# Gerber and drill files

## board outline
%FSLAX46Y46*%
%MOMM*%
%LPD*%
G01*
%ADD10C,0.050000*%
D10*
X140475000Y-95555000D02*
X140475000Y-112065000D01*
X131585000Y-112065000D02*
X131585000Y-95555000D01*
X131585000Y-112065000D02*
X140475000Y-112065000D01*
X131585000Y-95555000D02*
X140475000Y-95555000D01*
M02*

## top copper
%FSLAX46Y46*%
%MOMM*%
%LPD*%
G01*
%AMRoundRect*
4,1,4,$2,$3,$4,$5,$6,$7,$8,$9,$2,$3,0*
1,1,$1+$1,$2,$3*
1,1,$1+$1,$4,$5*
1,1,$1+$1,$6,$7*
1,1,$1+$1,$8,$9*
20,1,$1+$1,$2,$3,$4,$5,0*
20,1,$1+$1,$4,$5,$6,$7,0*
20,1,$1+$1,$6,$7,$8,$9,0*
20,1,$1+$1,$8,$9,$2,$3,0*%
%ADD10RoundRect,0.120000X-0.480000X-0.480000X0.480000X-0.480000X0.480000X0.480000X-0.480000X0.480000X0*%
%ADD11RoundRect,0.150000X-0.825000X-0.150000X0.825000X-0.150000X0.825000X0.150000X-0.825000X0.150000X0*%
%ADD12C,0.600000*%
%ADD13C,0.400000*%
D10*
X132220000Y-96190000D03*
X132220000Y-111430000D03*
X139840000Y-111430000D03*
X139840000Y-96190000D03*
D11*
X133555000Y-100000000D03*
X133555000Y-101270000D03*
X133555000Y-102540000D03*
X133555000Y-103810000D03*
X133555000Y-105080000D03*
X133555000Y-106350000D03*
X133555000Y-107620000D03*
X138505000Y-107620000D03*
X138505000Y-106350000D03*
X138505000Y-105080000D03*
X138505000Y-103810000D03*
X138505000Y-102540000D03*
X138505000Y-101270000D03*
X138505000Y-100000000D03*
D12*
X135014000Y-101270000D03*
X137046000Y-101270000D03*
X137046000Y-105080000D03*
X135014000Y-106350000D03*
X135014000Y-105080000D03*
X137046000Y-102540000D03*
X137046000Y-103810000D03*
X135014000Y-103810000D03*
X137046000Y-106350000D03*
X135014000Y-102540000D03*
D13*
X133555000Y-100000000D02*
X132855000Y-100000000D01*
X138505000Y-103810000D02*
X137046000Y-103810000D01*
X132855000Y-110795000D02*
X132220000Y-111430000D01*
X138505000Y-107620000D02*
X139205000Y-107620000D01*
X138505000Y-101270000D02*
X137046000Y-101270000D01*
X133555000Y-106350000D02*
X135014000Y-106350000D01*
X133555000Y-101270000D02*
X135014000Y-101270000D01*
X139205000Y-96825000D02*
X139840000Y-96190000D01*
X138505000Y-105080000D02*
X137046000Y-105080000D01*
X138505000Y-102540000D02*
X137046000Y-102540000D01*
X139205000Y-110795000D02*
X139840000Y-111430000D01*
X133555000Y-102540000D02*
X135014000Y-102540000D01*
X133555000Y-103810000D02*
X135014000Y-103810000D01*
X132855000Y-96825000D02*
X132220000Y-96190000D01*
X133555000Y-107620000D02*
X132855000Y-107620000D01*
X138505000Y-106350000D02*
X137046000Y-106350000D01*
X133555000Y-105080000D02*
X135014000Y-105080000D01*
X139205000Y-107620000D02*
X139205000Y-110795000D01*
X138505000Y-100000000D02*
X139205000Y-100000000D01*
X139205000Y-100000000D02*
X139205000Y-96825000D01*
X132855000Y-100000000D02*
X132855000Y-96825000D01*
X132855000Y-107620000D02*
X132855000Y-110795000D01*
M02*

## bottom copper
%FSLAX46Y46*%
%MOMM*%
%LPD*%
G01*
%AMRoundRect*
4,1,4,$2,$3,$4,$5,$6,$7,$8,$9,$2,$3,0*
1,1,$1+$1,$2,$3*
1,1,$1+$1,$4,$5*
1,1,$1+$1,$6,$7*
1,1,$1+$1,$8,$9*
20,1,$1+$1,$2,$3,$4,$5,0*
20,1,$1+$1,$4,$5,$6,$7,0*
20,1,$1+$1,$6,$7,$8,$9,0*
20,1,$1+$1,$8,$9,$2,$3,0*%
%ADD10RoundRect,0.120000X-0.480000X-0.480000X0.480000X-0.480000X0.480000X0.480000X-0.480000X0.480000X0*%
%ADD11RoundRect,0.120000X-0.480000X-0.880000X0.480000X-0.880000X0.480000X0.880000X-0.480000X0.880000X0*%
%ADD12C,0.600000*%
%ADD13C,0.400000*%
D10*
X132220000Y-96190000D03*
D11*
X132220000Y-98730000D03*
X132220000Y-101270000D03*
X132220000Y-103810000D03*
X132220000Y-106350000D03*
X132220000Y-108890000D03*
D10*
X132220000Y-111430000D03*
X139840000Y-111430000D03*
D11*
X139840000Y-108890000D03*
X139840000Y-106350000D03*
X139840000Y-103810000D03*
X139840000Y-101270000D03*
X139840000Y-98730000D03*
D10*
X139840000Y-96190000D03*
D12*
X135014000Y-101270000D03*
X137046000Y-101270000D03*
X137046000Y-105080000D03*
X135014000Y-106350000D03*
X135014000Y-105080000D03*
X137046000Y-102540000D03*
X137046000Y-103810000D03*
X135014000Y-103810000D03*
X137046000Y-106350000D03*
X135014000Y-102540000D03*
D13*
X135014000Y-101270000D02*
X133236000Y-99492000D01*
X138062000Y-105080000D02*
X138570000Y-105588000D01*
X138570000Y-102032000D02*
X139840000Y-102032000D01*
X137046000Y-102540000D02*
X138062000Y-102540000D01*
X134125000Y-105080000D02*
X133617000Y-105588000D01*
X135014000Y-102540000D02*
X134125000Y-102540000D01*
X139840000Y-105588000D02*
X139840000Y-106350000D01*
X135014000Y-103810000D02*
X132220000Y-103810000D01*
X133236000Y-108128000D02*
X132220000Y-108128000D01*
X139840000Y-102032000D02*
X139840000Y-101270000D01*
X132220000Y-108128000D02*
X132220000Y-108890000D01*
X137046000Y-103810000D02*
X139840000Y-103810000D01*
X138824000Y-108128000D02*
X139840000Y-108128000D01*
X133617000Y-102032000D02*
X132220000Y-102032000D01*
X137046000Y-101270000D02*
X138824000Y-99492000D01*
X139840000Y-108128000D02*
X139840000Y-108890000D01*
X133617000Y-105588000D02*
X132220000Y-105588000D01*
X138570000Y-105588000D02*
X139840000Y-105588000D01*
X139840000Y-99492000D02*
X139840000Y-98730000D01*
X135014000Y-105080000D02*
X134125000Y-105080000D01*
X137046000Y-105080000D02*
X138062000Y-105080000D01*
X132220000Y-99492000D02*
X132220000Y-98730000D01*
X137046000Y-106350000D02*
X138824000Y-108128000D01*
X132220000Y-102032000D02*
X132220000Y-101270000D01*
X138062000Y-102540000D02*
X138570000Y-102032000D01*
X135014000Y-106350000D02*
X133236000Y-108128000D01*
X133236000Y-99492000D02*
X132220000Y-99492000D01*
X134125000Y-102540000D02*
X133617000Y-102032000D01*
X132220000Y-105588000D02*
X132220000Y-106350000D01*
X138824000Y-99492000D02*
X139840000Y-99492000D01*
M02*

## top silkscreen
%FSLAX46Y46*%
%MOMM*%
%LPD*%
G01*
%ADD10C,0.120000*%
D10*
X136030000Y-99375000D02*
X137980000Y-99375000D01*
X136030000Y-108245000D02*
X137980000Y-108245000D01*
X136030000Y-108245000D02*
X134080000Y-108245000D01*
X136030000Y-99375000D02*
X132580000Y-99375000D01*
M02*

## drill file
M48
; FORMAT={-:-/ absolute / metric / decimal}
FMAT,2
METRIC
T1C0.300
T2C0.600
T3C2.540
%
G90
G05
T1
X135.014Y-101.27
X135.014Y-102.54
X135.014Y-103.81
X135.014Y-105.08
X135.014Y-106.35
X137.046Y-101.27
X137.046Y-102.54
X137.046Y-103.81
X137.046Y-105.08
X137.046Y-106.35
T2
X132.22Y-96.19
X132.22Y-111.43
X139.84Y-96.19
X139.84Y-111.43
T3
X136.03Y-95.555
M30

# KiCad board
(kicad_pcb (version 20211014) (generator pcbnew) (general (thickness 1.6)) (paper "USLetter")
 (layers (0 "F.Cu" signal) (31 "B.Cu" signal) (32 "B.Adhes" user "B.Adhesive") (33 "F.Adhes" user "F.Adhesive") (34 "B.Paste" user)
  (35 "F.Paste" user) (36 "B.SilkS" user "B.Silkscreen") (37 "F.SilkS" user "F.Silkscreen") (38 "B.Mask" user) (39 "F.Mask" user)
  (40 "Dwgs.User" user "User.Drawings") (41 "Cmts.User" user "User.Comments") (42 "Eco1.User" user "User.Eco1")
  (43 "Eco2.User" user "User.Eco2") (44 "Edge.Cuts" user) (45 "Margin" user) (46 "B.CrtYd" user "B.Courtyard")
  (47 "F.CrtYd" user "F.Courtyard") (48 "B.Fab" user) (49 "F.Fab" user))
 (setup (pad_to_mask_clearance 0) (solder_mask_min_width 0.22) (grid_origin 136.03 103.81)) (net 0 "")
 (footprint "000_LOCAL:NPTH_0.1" (layer "F.Cu") (at 136.03 95.555)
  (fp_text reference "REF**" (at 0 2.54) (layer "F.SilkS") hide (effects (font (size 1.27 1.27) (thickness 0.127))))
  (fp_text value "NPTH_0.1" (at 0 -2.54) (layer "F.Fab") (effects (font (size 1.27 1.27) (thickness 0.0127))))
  (pad "" np_thru_hole circle locked (at 0 0) (size 2.54 2.54) (drill 2.54) (layers *.Cu *.Mask)))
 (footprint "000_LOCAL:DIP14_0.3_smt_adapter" (layer "F.Cu") (at 136.03 103.81)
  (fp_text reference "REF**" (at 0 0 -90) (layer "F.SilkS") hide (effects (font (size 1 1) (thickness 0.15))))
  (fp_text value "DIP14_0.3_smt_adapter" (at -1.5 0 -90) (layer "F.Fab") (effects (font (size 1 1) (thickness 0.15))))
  (pad "1" thru_hole roundrect locked (at -3.81 -7.62) (size 1.2 1.2) (drill 0.6) (layers *.Cu *.Mask) (roundrect_rratio 0.1))
  (pad "2" smd roundrect locked (at -3.81 -5.08) (size 1.2 2) (layers "B.Cu" "B.Mask") (roundrect_rratio 0.1))
  (pad "3" smd roundrect locked (at -3.81 -2.54) (size 1.2 2) (layers "B.Cu" "B.Mask") (roundrect_rratio 0.1))
  (pad "4" smd roundrect locked (at -3.81 0) (size 1.2 2) (layers "B.Cu" "B.Mask") (roundrect_rratio 0.1))
  (pad "5" smd roundrect locked (at -3.81 2.54) (size 1.2 2) (layers "B.Cu" "B.Mask") (roundrect_rratio 0.1))
  (pad "6" smd roundrect locked (at -3.81 5.08) (size 1.2 2) (layers "B.Cu" "B.Mask") (roundrect_rratio 0.1))
  (pad "7" thru_hole roundrect locked (at -3.81 7.62) (size 1.2 1.2) (drill 0.6) (layers *.Cu *.Mask) (roundrect_rratio 0.1))
  (pad "8" thru_hole roundrect locked (at 3.81 7.62) (size 1.2 1.2) (drill 0.6) (layers *.Cu *.Mask) (roundrect_rratio 0.1))
  (pad "9" smd roundrect locked (at 3.81 5.08) (size 1.2 2) (layers "B.Cu" "B.Mask") (roundrect_rratio 0.1))
  (pad "10" smd roundrect locked (at 3.81 2.54) (size 1.2 2) (layers "B.Cu" "B.Mask") (roundrect_rratio 0.1))
  (pad "11" smd roundrect locked (at 3.81 0) (size 1.2 2) (layers "B.Cu" "B.Mask") (roundrect_rratio 0.1))
  (pad "12" smd roundrect locked (at 3.81 -2.54) (size 1.2 2) (layers "B.Cu" "B.Mask") (roundrect_rratio 0.1))
  (pad "13" smd roundrect locked (at 3.81 -5.08) (size 1.2 2) (layers "B.Cu" "B.Mask") (roundrect_rratio 0.1))
  (pad "14" thru_hole roundrect locked (at 3.81 -7.62) (size 1.2 1.2) (drill 0.6) (layers *.Cu *.Mask) (roundrect_rratio 0.1)))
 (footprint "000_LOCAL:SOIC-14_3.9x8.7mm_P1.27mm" (layer "F.Cu") (at 136.03 103.81)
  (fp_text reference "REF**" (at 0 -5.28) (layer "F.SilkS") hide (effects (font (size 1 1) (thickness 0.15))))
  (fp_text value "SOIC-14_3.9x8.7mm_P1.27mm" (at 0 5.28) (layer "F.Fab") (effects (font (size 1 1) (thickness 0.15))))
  (fp_line (start 0 -4.435) (end 1.95 -4.435) (layer "F.SilkS") (width 0.12))
  (fp_line (start 0 4.435) (end 1.95 4.435) (layer "F.SilkS") (width 0.12))
  (fp_line (start 0 4.435) (end -1.95 4.435) (layer "F.SilkS") (width 0.12))
  (fp_line (start 0 -4.435) (end -3.45 -4.435) (layer "F.SilkS") (width 0.12))
  (pad "1" smd roundrect locked (at -2.475 -3.81) (size 1.95 0.6) (layers "F.Cu" "F.Paste" "F.Mask") (roundrect_rratio 0.25))
  (pad "2" smd roundrect locked (at -2.475 -2.54) (size 1.95 0.6) (layers "F.Cu" "F.Paste" "F.Mask") (roundrect_rratio 0.25))
  (pad "3" smd roundrect locked (at -2.475 -1.27) (size 1.95 0.6) (layers "F.Cu" "F.Paste" "F.Mask") (roundrect_rratio 0.25))
  (pad "4" smd roundrect locked (at -2.475 0) (size 1.95 0.6) (layers "F.Cu" "F.Paste" "F.Mask") (roundrect_rratio 0.25))
  (pad "5" smd roundrect locked (at -2.475 1.27) (size 1.95 0.6) (layers "F.Cu" "F.Paste" "F.Mask") (roundrect_rratio 0.25))
  (pad "6" smd roundrect locked (at -2.475 2.54) (size 1.95 0.6) (layers "F.Cu" "F.Paste" "F.Mask") (roundrect_rratio 0.25))
  (pad "7" smd roundrect locked (at -2.475 3.81) (size 1.95 0.6) (layers "F.Cu" "F.Paste" "F.Mask") (roundrect_rratio 0.25))
  (pad "8" smd roundrect locked (at 2.475 3.81) (size 1.95 0.6) (layers "F.Cu" "F.Paste" "F.Mask") (roundrect_rratio 0.25))
  (pad "9" smd roundrect locked (at 2.475 2.54) (size 1.95 0.6) (layers "F.Cu" "F.Paste" "F.Mask") (roundrect_rratio 0.25))
  (pad "10" smd roundrect locked (at 2.475 1.27) (size 1.95 0.6) (layers "F.Cu" "F.Paste" "F.Mask") (roundrect_rratio 0.25))
  (pad "11" smd roundrect locked (at 2.475 0) (size 1.95 0.6) (layers "F.Cu" "F.Paste" "F.Mask") (roundrect_rratio 0.25))
  (pad "12" smd roundrect locked (at 2.475 -1.27) (size 1.95 0.6) (layers "F.Cu" "F.Paste" "F.Mask") (roundrect_rratio 0.25))
  (pad "13" smd roundrect locked (at 2.475 -2.54) (size 1.95 0.6) (layers "F.Cu" "F.Paste" "F.Mask") (roundrect_rratio 0.25))
  (pad "14" smd roundrect locked (at 2.475 -3.81) (size 1.95 0.6) (layers "F.Cu" "F.Paste" "F.Mask") (roundrect_rratio 0.25)))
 (gr_line (start 140.475 95.555) (end 140.475 112.065) (layer "Edge.Cuts") (width 0.05))
 (gr_line (start 131.585 112.065) (end 131.585 95.555) (layer "Edge.Cuts") (width 0.05))
 (gr_line (start 131.585 112.065) (end 140.475 112.065) (layer "Edge.Cuts") (width 0.05))
 (gr_line (start 131.585 95.555) (end 140.475 95.555) (layer "Edge.Cuts") (width 0.05))
 (segment (start 133.555 100) (end 132.855 100) (width 0.4) (layer "F.Cu") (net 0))
 (segment (start 138.505 103.81) (end 137.046 103.81) (width 0.4) (layer "F.Cu") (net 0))
 (segment (start 132.855 110.795) (end 132.22 111.43) (width 0.4) (layer "F.Cu") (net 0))
 (segment (start 138.505 107.62) (end 139.205 107.62) (width 0.4) (layer "F.Cu") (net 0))
 (segment (start 138.505 101.27) (end 137.046 101.27) (width 0.4) (layer "F.Cu") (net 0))
 (segment (start 133.555 106.35) (end 135.014 106.35) (width 0.4) (layer "F.Cu") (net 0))
 (segment (start 133.555 101.27) (end 135.014 101.27) (width 0.4) (layer "F.Cu") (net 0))
 (segment (start 139.205 96.825) (end 139.84 96.19) (width 0.4) (layer "F.Cu") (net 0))
 (segment (start 138.505 105.08) (end 137.046 105.08) (width 0.4) (layer "F.Cu") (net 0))
 (segment (start 138.505 102.54) (end 137.046 102.54) (width 0.4) (layer "F.Cu") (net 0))
 (segment (start 139.205 110.795) (end 139.84 111.43) (width 0.4) (layer "F.Cu") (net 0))
 (segment (start 133.555 102.54) (end 135.014 102.54) (width 0.4) (layer "F.Cu") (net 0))
 (segment (start 133.555 103.81) (end 135.014 103.81) (width 0.4) (layer "F.Cu") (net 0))
 (segment (start 132.855 96.825) (end 132.22 96.19) (width 0.4) (layer "F.Cu") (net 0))
 (segment (start 133.555 107.62) (end 132.855 107.62) (width 0.4) (layer "F.Cu") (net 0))
 (segment (start 138.505 106.35) (end 137.046 106.35) (width 0.4) (layer "F.Cu") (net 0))
 (segment (start 133.555 105.08) (end 135.014 105.08) (width 0.4) (layer "F.Cu") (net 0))
 (segment (start 139.205 107.62) (end 139.205 110.795) (width 0.4) (layer "F.Cu") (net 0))
 (segment (start 138.505 100) (end 139.205 100) (width 0.4) (layer "F.Cu") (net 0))
 (segment (start 139.205 100) (end 139.205 96.825) (width 0.4) (layer "F.Cu") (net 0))
 (segment (start 132.855 100) (end 132.855 96.825) (width 0.4) (layer "F.Cu") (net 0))
 (segment (start 132.855 107.62) (end 132.855 110.795) (width 0.4) (layer "F.Cu") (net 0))
 (via (at 135.014 101.27) (size 0.6) (drill 0.3) (layers "F.Cu" "B.Cu") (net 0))
 (via (at 137.046 101.27) (size 0.6) (drill 0.3) (layers "F.Cu" "B.Cu") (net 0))
 (via (at 137.046 105.08) (size 0.6) (drill 0.3) (layers "F.Cu" "B.Cu") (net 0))
 (via (at 135.014 106.35) (size 0.6) (drill 0.3) (layers "F.Cu" "B.Cu") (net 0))
 (via (at 135.014 105.08) (size 0.6) (drill 0.3) (layers "F.Cu" "B.Cu") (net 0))
 (via (at 137.046 102.54) (size 0.6) (drill 0.3) (layers "F.Cu" "B.Cu") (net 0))
 (via (at 137.046 103.81) (size 0.6) (drill 0.3) (layers "F.Cu" "B.Cu") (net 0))
 (via (at 135.014 103.81) (size 0.6) (drill 0.3) (layers "F.Cu" "B.Cu") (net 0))
 (via (at 137.046 106.35) (size 0.6) (drill 0.3) (layers "F.Cu" "B.Cu") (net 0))
 (via (at 135.014 102.54) (size 0.6) (drill 0.3) (layers "F.Cu" "B.Cu") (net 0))
 (segment (start 135.014 101.27) (end 133.236 99.492) (width 0.4) (layer "B.Cu") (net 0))
 (segment (start 138.062 105.08) (end 138.57 105.588) (width 0.4) (layer "B.Cu") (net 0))
 (segment (start 138.57 102.032) (end 139.84 102.032) (width 0.4) (layer "B.Cu") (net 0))
 (segment (start 137.046 102.54) (end 138.062 102.54) (width 0.4) (layer "B.Cu") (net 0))
 (segment (start 134.125 105.08) (end 133.617 105.588) (width 0.4) (layer "B.Cu") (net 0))
 (segment (start 135.014 102.54) (end 134.125 102.54) (width 0.4) (layer "B.Cu") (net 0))
 (segment (start 139.84 105.588) (end 139.84 106.35) (width 0.4) (layer "B.Cu") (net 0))
 (segment (start 135.014 103.81) (end 132.22 103.81) (width 0.4) (layer "B.Cu") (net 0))
 (segment (start 133.236 108.128) (end 132.22 108.128) (width 0.4) (layer "B.Cu") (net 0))
 (segment (start 139.84 102.032) (end 139.84 101.27) (width 0.4) (layer "B.Cu") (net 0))
 (segment (start 132.22 108.128) (end 132.22 108.89) (width 0.4) (layer "B.Cu") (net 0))
 (segment (start 137.046 103.81) (end 139.84 103.81) (width 0.4) (layer "B.Cu") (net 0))
 (segment (start 138.824 108.128) (end 139.84 108.128) (width 0.4) (layer "B.Cu") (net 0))
 (segment (start 133.617 102.032) (end 132.22 102.032) (width 0.4) (layer "B.Cu") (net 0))
 (segment (start 137.046 101.27) (end 138.824 99.492) (width 0.4) (layer "B.Cu") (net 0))
 (segment (start 139.84 108.128) (end 139.84 108.89) (width 0.4) (layer "B.Cu") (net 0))
 (segment (start 133.617 105.588) (end 132.22 105.588) (width 0.4) (layer "B.Cu") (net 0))
 (segment (start 138.57 105.588) (end 139.84 105.588) (width 0.4) (layer "B.Cu") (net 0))
 (segment (start 139.84 99.492) (end 139.84 98.73) (width 0.4) (layer "B.Cu") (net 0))
 (segment (start 135.014 105.08) (end 134.125 105.08) (width 0.4) (layer "B.Cu") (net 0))
 (segment (start 137.046 105.08) (end 138.062 105.08) (width 0.4) (layer "B.Cu") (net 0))
 (segment (start 132.22 99.492) (end 132.22 98.73) (width 0.4) (layer "B.Cu") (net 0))
 (segment (start 137.046 106.35) (end 138.824 108.128) (width 0.4) (layer "B.Cu") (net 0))
 (segment (start 132.22 102.032) (end 132.22 101.27) (width 0.4) (layer "B.Cu") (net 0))
 (segment (start 138.062 102.54) (end 138.57 102.032) (width 0.4) (layer "B.Cu") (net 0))
 (segment (start 135.014 106.35) (end 133.236 108.128) (width 0.4) (layer "B.Cu") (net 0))
 (segment (start 133.236 99.492) (end 132.22 99.492) (width 0.4) (layer "B.Cu") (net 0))
 (segment (start 134.125 102.54) (end 133.617 102.032) (width 0.4) (layer "B.Cu") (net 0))
 (segment (start 132.22 105.588) (end 132.22 106.35) (width 0.4) (layer "B.Cu") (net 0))
 (segment (start 138.824 99.492) (end 139.84 99.492) (width 0.4) (layer "B.Cu") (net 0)))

